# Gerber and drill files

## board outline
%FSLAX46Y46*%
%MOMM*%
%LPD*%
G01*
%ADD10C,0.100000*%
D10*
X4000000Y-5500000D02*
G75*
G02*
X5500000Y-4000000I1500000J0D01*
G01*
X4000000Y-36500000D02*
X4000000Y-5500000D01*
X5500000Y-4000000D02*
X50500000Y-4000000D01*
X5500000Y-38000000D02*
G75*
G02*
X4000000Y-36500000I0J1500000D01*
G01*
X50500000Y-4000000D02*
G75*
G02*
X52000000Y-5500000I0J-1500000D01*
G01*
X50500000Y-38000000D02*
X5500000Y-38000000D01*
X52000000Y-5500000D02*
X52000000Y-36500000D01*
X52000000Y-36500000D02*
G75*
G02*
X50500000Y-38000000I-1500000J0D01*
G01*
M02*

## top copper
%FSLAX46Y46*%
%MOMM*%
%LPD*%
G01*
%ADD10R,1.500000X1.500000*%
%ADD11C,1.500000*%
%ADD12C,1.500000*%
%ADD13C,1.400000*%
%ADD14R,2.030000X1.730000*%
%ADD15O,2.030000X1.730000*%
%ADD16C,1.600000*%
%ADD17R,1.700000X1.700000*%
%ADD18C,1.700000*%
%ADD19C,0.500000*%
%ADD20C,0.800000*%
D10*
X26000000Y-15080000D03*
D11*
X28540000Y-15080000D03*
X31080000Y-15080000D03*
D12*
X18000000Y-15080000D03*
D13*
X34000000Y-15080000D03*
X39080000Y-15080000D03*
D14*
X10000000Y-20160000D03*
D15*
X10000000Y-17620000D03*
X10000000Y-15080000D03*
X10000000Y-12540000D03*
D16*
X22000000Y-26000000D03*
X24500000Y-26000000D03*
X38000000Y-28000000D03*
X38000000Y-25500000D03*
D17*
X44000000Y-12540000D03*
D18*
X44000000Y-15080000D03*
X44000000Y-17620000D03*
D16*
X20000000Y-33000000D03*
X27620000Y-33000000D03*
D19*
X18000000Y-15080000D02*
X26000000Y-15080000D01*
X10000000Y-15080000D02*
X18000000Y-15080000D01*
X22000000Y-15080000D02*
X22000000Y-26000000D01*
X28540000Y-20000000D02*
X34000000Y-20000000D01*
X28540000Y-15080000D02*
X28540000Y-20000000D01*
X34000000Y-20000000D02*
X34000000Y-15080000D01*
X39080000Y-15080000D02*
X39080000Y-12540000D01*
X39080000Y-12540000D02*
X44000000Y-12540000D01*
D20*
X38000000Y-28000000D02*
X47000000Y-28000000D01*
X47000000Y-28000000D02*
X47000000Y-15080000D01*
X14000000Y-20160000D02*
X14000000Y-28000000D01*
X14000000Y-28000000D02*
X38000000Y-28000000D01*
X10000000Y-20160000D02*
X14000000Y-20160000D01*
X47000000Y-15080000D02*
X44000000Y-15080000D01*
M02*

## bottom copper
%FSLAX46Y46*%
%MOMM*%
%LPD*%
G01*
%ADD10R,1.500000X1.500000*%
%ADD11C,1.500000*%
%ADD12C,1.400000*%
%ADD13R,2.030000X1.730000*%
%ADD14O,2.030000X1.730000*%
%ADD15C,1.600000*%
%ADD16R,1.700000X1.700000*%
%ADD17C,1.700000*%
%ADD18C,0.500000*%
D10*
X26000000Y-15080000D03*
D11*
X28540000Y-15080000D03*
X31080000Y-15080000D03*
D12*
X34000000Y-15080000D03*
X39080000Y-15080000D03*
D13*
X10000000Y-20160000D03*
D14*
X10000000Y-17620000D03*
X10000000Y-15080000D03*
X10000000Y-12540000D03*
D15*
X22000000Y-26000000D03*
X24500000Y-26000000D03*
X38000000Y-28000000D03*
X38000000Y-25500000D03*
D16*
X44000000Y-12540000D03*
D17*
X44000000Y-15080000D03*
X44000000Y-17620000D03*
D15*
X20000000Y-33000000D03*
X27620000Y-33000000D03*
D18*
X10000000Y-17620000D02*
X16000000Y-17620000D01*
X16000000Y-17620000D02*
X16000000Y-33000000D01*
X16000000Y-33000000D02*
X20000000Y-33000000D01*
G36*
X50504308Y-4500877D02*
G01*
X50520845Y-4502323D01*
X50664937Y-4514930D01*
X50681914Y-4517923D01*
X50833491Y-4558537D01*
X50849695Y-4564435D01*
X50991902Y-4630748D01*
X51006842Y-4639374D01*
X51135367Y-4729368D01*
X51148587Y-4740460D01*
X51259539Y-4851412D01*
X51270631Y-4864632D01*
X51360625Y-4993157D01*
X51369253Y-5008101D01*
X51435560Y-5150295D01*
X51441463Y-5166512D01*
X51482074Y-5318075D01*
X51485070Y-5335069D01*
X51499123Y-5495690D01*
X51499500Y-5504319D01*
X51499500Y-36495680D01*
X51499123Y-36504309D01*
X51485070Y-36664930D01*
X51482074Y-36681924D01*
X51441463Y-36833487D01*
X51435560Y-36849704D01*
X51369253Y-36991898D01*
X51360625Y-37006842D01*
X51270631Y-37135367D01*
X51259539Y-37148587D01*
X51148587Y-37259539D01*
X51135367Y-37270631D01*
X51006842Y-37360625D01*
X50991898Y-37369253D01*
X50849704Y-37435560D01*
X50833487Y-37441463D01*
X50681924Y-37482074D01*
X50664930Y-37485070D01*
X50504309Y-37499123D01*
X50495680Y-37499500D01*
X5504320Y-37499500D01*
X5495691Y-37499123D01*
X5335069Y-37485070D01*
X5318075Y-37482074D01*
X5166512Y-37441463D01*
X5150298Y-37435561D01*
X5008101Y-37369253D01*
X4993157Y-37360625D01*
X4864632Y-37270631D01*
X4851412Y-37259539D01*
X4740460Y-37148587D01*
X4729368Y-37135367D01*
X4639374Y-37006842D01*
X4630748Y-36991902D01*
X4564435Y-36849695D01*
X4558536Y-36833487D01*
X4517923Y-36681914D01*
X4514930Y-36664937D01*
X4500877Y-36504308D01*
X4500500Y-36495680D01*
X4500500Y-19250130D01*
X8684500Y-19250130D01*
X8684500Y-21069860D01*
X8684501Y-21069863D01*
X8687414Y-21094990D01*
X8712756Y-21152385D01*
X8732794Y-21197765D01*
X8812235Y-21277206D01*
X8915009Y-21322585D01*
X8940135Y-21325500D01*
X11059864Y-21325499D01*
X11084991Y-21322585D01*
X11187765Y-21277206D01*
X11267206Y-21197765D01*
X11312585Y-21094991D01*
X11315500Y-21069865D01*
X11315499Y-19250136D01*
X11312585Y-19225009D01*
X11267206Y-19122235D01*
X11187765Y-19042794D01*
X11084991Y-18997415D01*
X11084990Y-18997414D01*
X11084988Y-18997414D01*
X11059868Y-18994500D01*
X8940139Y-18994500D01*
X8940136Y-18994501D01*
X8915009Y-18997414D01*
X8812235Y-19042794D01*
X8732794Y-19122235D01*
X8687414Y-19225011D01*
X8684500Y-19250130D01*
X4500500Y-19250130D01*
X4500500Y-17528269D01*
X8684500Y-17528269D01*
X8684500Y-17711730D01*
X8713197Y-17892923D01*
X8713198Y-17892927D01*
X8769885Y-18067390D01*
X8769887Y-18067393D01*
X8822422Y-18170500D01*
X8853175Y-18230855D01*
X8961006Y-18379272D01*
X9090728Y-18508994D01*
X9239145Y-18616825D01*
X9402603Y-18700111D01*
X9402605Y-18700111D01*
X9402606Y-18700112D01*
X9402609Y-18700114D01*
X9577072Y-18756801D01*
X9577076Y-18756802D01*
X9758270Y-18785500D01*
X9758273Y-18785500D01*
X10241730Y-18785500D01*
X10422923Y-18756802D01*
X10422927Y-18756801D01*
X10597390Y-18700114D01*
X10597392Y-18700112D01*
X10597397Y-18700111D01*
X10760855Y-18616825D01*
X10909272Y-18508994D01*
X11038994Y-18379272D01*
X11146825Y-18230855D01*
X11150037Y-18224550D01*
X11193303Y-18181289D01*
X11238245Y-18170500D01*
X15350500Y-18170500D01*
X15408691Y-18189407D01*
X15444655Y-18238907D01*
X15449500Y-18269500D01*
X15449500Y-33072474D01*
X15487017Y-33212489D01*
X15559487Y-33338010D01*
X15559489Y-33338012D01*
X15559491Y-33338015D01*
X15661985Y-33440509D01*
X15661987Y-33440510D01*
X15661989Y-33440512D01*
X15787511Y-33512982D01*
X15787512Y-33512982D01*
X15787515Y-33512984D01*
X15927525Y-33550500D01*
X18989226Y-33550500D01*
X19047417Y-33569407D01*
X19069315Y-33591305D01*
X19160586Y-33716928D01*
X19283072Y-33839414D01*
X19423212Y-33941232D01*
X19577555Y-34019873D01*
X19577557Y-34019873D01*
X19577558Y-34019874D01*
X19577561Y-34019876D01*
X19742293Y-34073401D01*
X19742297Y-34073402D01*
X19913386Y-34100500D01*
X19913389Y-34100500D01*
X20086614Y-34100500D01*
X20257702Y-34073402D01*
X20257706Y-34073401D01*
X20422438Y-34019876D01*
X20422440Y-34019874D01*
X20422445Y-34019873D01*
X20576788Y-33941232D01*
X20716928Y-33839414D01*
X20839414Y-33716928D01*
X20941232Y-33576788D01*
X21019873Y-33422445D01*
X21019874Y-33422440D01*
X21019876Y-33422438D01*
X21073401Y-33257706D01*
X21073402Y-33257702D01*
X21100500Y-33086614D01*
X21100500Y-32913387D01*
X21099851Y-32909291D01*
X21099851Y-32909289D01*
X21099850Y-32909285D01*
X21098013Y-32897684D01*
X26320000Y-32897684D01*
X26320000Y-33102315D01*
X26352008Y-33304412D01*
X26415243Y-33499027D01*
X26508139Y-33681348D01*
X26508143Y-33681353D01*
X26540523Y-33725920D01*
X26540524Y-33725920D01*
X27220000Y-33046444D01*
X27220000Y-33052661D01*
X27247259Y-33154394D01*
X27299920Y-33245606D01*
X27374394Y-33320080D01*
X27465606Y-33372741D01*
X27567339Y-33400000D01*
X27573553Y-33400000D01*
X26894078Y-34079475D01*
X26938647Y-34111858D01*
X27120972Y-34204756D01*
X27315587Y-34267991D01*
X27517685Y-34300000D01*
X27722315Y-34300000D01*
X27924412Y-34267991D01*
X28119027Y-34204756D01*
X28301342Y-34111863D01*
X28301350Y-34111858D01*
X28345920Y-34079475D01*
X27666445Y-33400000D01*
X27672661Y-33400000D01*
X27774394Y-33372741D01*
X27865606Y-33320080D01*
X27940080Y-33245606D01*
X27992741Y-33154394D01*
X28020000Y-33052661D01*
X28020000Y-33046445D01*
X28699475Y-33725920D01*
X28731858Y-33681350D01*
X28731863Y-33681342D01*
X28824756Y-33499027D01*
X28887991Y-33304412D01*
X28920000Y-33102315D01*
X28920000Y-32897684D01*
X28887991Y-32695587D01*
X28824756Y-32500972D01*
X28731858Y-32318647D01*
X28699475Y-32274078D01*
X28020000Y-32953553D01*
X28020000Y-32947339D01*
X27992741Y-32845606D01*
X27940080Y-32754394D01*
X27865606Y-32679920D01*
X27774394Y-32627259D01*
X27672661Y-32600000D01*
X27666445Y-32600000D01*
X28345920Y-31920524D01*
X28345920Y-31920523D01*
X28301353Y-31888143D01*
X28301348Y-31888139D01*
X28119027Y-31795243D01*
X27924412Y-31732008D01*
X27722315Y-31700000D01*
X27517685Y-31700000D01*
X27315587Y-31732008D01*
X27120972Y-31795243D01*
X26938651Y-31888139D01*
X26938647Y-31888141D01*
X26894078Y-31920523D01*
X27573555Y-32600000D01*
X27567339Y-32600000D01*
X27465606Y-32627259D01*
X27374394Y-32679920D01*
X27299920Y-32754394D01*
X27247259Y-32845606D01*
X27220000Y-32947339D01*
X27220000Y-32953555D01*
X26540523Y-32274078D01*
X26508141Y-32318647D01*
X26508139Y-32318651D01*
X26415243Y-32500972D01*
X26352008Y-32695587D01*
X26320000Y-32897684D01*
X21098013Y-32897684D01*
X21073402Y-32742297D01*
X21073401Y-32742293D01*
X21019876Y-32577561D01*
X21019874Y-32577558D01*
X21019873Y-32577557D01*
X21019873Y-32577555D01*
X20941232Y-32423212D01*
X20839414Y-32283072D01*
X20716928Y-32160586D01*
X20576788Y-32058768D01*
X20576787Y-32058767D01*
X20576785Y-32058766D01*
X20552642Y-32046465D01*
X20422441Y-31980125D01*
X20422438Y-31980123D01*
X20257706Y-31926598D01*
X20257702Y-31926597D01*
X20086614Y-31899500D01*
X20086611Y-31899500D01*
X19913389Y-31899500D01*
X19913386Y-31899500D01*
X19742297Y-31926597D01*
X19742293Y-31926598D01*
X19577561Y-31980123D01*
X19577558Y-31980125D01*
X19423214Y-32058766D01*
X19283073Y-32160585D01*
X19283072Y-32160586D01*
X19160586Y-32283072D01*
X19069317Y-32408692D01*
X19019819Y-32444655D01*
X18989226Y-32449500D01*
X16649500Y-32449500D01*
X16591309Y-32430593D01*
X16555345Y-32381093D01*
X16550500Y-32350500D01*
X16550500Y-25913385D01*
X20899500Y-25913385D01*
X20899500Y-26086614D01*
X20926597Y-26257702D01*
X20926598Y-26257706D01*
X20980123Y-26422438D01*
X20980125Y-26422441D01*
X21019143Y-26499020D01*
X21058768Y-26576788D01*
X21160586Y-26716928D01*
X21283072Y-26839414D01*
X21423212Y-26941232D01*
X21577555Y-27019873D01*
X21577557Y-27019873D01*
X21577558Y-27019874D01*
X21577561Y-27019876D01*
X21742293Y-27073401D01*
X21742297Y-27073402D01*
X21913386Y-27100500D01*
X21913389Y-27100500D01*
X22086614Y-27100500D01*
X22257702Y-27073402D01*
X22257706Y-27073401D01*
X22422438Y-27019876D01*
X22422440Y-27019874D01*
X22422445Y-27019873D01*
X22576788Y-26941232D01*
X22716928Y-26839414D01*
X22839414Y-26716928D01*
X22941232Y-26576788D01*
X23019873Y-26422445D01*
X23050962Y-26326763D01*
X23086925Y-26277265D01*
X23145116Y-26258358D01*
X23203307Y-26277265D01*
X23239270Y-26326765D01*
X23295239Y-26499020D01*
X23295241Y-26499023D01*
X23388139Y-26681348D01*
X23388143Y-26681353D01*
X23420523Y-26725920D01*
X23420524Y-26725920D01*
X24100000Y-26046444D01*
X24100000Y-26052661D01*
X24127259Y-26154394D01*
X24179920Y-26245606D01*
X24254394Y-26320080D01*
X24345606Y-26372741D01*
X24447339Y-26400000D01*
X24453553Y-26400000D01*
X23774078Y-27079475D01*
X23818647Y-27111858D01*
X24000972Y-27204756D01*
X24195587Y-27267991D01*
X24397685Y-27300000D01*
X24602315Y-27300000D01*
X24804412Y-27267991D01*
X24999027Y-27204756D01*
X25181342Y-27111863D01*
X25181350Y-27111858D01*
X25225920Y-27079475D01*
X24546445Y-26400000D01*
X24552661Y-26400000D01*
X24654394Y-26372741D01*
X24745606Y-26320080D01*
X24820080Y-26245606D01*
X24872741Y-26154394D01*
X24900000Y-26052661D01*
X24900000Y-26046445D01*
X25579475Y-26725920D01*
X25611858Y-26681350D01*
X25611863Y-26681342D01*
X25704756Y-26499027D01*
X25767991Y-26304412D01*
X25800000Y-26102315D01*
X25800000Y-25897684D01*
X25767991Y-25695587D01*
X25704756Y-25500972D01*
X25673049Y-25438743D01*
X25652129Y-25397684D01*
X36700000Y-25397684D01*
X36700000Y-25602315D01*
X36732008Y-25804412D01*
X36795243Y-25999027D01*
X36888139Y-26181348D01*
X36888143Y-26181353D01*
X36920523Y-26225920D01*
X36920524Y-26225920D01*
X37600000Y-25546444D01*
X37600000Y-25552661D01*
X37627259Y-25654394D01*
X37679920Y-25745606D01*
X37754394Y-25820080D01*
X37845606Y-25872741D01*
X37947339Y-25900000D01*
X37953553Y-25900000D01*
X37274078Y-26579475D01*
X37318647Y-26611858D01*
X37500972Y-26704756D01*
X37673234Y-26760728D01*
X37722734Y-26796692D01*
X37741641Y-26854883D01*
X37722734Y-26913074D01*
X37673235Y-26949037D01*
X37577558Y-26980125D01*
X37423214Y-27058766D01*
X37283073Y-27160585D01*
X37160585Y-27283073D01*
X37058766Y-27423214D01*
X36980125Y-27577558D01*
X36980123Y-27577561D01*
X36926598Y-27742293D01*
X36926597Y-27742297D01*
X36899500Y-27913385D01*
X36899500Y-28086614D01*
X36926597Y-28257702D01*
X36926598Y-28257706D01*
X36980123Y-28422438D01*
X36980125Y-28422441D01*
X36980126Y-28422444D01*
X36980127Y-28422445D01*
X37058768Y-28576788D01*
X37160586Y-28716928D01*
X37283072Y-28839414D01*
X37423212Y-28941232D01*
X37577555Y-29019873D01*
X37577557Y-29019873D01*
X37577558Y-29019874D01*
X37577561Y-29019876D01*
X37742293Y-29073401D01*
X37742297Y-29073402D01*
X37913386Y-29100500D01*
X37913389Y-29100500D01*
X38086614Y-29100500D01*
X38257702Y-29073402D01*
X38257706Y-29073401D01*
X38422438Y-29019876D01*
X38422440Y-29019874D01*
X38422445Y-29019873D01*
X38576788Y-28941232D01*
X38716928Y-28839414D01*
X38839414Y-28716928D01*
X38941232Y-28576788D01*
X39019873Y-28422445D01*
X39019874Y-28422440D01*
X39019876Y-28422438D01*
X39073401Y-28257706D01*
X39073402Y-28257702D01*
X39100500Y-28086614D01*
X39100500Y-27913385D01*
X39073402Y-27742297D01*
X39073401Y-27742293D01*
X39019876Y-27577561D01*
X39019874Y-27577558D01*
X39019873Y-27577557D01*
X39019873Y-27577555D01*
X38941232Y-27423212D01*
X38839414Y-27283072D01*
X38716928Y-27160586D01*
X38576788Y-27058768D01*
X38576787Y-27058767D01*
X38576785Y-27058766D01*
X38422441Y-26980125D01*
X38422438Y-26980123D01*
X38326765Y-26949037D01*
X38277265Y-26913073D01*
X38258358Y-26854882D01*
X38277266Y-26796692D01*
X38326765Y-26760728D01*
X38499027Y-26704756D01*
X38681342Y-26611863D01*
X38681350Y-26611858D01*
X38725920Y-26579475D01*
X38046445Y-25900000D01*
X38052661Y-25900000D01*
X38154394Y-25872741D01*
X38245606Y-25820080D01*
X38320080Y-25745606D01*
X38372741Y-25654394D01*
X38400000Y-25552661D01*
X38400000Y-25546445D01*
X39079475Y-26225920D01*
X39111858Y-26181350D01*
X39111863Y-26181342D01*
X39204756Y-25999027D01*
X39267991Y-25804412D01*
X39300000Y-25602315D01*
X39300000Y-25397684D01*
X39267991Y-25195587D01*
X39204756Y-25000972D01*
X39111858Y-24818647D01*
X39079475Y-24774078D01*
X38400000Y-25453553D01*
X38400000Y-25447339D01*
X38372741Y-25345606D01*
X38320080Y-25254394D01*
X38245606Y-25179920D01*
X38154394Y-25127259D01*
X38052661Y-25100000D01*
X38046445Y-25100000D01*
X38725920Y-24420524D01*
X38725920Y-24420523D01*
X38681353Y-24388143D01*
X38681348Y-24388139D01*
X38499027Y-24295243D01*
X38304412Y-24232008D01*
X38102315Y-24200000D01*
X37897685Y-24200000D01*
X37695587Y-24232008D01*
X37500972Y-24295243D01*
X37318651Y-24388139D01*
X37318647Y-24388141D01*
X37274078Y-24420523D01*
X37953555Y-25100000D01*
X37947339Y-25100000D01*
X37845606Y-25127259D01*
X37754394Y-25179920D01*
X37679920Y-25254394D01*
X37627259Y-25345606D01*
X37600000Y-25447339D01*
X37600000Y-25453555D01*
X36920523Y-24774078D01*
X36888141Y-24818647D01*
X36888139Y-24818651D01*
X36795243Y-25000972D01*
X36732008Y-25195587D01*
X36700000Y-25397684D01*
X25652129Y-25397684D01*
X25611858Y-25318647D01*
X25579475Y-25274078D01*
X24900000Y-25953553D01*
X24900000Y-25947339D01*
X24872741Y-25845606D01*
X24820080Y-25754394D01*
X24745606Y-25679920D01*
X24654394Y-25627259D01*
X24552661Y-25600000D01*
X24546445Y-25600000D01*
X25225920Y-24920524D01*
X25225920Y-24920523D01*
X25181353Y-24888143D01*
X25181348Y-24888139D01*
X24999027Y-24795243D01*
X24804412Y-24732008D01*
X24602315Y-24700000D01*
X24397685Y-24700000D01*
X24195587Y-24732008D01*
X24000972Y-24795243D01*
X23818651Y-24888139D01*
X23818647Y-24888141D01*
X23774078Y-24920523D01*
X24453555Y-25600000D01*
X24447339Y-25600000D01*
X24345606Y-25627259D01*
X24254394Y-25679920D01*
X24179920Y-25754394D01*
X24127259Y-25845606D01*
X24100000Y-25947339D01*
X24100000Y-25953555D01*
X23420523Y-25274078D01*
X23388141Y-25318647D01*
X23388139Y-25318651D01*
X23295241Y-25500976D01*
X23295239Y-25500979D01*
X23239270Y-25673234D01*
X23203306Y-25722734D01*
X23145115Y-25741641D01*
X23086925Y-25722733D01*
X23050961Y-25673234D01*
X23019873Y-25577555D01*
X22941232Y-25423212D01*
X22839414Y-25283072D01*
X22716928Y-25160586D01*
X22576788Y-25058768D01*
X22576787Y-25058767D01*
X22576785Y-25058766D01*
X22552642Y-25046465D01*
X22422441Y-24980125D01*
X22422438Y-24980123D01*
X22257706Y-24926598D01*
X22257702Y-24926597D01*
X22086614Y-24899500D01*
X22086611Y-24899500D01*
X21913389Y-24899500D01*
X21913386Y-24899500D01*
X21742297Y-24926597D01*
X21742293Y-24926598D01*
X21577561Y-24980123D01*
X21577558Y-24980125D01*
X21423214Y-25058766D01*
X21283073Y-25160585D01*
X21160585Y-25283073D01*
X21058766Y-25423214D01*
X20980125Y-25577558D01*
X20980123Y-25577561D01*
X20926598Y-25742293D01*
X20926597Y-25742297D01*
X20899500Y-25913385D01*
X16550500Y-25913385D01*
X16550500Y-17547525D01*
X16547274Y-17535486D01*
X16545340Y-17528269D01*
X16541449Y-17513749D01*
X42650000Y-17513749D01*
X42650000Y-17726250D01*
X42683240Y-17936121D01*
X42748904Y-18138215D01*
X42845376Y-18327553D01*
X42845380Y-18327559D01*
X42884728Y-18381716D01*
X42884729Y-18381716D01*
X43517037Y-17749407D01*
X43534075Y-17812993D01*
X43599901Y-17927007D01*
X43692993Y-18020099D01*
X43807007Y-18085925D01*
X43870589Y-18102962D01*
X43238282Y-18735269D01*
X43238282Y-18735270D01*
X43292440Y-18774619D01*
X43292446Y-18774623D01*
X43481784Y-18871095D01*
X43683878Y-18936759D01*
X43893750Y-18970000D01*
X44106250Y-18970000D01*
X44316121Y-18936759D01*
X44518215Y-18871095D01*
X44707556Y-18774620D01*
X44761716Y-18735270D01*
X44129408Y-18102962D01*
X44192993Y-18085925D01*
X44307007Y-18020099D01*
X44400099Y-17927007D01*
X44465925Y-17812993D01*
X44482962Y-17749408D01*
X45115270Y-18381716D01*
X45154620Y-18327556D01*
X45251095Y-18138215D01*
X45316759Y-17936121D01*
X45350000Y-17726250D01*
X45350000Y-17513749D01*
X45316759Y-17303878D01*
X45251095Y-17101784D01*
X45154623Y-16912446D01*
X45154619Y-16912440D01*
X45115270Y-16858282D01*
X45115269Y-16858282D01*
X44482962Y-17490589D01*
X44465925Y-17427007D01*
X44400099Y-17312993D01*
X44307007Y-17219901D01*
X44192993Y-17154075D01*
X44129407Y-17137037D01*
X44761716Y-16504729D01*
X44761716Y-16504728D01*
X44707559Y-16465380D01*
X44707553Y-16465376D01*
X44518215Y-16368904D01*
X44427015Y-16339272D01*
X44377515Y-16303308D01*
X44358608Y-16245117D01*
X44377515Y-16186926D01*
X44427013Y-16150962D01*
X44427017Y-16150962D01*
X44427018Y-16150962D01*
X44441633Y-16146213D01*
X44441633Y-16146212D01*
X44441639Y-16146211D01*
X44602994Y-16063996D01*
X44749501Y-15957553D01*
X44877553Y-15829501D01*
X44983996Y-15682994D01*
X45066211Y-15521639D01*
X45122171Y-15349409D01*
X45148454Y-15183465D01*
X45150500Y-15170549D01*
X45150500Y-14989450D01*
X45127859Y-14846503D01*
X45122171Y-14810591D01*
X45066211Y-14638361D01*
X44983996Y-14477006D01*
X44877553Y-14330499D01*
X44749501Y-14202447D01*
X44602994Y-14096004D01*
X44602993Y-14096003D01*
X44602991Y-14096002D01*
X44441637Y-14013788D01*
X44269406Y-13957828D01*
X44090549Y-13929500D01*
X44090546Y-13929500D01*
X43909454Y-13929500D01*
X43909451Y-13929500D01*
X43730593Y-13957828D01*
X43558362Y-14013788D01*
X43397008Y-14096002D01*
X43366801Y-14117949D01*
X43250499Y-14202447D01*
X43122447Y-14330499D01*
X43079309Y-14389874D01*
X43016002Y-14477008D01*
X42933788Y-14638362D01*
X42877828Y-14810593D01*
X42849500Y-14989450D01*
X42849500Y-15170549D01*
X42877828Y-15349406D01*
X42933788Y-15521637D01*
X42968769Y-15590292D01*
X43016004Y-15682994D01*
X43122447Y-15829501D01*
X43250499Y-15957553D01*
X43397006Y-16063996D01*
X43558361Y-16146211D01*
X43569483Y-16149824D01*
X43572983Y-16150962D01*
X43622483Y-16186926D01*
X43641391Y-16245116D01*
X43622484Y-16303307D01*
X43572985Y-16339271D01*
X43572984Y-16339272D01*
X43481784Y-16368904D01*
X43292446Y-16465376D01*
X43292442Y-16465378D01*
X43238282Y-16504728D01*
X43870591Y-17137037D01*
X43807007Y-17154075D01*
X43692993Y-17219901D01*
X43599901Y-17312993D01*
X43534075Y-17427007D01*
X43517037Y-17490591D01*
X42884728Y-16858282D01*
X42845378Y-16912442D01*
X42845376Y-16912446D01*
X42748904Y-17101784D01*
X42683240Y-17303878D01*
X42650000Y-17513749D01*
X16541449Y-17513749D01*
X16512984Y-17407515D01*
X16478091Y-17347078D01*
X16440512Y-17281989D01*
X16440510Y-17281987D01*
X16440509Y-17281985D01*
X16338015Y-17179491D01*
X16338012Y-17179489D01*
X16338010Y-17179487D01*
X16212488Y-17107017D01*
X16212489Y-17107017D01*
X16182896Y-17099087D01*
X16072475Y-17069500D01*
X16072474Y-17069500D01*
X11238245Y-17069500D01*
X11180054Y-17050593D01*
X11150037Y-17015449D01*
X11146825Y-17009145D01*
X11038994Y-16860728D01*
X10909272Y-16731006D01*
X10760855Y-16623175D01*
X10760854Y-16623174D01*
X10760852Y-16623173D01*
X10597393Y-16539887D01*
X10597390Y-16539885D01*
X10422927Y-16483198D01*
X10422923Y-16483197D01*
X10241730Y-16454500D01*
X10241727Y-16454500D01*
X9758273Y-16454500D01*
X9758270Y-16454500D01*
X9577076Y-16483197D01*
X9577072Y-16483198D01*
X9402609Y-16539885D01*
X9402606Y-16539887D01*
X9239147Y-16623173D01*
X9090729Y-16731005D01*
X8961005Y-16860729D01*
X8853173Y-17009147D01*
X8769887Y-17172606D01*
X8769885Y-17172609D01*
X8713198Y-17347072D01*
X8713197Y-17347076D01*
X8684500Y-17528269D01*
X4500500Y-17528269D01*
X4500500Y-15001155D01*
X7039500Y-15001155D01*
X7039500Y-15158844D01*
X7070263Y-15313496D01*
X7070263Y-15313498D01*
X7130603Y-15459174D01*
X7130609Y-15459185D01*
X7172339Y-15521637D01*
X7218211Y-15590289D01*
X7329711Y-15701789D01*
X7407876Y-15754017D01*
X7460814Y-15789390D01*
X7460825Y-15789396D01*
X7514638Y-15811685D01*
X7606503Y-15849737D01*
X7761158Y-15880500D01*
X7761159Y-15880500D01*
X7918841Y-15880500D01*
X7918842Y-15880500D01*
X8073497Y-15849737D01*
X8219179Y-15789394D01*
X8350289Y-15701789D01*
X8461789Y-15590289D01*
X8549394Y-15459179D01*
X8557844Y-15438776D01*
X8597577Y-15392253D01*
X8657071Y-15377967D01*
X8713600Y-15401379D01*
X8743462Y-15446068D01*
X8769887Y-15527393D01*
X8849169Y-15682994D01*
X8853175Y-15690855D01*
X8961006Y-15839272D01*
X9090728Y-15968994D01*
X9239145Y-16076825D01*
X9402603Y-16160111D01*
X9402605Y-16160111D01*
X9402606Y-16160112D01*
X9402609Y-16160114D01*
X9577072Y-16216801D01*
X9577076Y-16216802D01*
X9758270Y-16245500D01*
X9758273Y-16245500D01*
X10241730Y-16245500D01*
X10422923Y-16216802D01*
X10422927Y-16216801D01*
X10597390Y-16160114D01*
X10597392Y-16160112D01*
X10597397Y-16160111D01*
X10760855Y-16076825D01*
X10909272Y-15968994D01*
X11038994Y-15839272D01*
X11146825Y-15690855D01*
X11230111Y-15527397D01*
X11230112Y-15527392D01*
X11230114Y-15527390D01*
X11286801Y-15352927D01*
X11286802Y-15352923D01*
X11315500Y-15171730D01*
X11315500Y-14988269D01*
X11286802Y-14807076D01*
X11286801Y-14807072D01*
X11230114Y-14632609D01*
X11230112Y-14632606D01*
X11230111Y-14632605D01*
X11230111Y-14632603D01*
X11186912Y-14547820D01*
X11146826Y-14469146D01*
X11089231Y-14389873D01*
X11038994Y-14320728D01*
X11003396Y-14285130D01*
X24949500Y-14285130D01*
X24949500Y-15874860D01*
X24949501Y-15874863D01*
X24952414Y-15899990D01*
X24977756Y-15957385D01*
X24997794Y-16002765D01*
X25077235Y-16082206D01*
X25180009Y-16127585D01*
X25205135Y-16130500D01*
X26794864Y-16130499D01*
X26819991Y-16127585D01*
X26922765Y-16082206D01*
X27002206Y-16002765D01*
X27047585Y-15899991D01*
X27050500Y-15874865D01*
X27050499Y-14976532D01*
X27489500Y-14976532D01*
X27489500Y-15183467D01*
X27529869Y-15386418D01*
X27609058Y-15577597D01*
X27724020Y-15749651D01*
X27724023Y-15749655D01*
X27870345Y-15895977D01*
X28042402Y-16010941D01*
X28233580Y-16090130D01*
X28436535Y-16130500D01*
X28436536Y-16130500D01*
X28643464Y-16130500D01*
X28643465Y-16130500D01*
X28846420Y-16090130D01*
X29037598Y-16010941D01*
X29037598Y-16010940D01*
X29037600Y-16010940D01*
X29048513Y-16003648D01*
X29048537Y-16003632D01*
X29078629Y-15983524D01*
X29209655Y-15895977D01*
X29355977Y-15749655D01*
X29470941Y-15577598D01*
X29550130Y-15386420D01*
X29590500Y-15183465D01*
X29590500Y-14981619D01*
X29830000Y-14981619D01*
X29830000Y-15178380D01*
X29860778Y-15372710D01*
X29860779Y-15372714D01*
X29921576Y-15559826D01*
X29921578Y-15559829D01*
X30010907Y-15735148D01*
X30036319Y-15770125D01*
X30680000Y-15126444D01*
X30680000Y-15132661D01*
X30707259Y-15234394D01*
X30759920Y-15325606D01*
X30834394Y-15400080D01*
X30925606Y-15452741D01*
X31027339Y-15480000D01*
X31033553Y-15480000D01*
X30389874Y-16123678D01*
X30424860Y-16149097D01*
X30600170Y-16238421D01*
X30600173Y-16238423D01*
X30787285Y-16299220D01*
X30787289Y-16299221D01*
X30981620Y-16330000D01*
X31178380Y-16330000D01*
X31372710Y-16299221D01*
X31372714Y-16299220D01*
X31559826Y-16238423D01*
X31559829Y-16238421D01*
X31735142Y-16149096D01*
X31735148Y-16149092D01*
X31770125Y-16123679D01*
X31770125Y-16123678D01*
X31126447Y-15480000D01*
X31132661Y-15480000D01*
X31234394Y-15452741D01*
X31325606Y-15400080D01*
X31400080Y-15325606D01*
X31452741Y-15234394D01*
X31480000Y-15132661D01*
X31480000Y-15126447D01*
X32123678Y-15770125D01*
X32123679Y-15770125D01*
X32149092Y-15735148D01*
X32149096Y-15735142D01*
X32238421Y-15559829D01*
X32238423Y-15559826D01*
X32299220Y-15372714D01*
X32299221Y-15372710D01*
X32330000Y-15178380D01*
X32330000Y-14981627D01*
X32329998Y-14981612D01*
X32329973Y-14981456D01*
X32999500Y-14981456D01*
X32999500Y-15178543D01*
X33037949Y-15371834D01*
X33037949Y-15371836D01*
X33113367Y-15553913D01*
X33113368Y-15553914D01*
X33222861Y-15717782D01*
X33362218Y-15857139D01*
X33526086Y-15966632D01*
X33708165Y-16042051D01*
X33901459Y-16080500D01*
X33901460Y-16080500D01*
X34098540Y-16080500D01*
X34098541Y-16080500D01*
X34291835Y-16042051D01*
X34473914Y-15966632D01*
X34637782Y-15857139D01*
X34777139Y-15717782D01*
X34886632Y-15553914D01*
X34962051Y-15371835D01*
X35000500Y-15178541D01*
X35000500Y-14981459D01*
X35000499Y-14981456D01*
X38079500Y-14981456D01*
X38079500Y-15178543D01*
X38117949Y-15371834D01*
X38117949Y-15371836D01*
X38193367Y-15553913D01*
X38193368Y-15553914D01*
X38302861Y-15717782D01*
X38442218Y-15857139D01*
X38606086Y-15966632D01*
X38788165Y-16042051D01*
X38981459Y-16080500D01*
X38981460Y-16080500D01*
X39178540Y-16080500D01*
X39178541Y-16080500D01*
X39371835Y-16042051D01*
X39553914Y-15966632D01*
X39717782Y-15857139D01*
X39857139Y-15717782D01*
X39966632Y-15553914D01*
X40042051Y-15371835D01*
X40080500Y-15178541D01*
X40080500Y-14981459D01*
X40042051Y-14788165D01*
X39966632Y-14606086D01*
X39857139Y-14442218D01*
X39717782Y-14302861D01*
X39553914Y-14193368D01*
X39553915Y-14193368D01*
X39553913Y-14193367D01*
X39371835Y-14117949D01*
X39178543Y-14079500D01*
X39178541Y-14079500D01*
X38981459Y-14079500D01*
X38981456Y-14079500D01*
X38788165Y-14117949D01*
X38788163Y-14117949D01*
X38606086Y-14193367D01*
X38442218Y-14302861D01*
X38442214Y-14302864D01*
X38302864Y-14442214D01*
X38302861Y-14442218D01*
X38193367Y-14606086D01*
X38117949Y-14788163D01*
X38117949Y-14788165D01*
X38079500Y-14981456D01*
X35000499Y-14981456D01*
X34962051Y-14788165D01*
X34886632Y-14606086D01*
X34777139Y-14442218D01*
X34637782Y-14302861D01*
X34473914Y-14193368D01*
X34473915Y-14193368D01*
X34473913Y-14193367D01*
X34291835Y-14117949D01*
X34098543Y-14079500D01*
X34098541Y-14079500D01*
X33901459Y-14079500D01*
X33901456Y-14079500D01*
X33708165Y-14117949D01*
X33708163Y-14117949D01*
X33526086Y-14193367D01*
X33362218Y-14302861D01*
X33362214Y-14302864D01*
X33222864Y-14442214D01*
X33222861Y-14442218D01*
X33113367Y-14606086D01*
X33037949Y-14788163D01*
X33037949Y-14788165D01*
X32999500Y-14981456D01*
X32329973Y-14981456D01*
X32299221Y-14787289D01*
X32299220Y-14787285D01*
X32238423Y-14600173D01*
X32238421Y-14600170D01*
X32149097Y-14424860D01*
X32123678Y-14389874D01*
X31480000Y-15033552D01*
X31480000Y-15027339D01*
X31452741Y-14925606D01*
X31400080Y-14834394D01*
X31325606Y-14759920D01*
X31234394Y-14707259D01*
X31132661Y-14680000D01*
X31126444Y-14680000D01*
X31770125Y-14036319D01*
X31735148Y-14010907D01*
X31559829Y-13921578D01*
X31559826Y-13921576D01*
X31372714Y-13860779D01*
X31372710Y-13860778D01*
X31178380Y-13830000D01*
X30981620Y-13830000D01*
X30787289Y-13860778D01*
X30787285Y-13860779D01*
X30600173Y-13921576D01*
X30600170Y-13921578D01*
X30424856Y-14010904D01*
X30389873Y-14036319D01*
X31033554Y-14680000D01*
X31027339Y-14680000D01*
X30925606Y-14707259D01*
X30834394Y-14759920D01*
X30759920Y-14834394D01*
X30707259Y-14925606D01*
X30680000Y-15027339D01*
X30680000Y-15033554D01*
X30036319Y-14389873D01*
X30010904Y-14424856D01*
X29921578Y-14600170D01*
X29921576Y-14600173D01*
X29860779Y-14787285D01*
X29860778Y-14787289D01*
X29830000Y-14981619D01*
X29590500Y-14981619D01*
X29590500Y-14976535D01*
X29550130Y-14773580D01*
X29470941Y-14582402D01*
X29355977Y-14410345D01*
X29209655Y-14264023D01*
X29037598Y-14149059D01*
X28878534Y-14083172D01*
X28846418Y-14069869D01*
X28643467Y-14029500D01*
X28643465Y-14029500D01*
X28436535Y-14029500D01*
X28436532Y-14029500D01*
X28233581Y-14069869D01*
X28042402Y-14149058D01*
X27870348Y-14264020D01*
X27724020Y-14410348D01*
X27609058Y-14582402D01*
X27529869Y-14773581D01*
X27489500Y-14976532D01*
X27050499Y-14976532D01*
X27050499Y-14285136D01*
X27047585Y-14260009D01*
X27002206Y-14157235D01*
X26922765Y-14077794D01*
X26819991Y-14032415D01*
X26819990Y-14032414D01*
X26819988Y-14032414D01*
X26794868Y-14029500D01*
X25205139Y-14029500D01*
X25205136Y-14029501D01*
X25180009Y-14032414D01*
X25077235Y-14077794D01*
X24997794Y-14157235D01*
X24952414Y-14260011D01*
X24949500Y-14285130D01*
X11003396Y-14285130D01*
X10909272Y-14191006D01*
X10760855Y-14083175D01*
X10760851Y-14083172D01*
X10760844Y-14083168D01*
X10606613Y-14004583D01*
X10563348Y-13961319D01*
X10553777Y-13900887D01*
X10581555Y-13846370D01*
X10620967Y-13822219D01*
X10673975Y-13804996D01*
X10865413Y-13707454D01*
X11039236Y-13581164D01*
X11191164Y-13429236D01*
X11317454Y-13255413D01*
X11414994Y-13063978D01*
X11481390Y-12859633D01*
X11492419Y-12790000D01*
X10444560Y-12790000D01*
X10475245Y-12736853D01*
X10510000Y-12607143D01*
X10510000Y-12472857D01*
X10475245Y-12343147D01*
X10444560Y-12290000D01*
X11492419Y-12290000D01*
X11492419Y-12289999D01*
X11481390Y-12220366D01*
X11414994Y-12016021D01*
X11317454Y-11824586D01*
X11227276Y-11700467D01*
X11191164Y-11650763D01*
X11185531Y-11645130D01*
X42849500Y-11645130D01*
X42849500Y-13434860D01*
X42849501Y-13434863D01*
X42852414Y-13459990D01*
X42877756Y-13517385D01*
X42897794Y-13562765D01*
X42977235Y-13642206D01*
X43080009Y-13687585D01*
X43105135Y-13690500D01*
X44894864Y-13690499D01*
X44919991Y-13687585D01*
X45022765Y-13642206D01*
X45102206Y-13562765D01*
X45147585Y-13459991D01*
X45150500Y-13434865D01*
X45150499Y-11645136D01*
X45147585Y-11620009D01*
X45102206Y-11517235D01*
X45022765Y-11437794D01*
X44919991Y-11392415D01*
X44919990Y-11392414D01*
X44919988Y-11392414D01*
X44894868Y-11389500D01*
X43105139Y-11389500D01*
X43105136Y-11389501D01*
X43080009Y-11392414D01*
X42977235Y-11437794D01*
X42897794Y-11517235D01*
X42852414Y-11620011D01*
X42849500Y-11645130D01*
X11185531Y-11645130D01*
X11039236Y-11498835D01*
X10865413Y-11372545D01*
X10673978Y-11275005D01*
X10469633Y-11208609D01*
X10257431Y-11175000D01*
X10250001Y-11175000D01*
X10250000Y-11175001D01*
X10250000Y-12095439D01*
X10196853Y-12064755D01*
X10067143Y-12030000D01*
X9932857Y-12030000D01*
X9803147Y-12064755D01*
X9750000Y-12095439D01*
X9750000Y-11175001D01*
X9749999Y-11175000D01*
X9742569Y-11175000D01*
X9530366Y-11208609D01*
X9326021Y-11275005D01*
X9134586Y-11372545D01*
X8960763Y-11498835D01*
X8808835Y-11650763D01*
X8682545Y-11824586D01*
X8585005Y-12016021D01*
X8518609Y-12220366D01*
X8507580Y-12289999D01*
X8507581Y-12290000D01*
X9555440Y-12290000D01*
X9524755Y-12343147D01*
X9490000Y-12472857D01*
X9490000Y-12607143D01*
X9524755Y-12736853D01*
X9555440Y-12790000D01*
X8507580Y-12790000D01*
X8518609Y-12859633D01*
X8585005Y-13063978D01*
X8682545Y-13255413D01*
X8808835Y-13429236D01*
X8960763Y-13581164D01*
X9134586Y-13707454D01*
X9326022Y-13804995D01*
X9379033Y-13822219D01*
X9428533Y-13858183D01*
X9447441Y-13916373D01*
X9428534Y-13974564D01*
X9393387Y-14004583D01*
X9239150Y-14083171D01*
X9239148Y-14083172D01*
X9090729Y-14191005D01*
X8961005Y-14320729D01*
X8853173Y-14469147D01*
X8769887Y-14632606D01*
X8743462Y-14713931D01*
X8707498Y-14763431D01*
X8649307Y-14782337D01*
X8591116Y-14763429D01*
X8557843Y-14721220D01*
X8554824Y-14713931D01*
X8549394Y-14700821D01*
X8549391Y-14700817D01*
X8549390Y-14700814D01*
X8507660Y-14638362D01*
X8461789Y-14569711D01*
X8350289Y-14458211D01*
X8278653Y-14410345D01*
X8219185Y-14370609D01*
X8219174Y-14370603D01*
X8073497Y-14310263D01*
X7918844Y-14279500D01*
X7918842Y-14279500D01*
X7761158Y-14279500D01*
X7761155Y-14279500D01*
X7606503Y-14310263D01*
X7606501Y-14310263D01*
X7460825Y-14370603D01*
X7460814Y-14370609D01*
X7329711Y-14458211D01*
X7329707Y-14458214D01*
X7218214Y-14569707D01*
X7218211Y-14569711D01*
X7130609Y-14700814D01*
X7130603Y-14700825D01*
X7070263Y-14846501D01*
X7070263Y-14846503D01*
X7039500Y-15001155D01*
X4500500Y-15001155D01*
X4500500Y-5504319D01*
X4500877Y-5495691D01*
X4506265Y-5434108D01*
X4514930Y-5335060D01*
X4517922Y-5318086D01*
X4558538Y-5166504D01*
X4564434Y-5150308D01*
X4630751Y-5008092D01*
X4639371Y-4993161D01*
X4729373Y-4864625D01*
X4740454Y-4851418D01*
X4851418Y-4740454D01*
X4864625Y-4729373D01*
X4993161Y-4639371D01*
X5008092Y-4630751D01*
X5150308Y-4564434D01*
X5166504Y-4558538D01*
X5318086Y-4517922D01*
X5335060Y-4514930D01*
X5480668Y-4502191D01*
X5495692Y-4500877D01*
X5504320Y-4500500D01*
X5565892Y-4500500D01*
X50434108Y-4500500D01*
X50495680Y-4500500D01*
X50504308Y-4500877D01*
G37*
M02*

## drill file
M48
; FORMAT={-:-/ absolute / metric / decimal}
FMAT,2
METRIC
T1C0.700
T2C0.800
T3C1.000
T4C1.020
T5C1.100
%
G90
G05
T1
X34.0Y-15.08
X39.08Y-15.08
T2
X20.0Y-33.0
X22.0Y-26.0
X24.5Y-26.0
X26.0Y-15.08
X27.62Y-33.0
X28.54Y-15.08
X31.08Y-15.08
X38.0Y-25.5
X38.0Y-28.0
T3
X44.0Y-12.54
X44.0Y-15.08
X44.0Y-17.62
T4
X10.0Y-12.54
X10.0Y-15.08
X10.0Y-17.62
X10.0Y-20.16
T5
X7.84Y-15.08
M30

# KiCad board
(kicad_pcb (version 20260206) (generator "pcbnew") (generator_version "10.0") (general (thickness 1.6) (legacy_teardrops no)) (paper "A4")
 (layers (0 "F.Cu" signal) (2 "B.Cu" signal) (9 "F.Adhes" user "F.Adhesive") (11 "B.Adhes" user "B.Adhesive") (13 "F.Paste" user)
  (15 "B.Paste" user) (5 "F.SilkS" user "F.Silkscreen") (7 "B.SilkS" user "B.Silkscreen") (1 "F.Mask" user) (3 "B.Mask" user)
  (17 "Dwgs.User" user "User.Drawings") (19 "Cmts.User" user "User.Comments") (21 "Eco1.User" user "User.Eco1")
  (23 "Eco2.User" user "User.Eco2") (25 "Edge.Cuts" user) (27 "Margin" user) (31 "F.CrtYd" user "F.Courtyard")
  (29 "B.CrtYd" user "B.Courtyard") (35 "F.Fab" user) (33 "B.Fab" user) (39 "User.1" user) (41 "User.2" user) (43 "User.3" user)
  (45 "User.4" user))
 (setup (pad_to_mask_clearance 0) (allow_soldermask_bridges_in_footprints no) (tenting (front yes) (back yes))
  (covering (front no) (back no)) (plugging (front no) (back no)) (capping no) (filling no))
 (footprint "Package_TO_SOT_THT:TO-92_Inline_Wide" (layer "F.Cu") (at 26 15.08)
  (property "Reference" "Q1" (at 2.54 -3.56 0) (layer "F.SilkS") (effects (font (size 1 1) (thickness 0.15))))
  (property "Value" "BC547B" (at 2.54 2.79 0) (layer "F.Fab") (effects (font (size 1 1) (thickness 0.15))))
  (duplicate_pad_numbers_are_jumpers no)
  (pad "1" thru_hole rect (at 0 0) (size 1.5 1.5) (drill 0.8) (layers "*.Cu" "*.Mask") (remove_unused_layers no) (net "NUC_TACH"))
  (pad "2" thru_hole circle (at 2.54 0) (size 1.5 1.5) (drill 0.8) (layers "*.Cu" "*.Mask") (remove_unused_layers no) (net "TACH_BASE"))
  (pad "3" thru_hole circle (at 5.08 0) (size 1.5 1.5) (drill 0.8) (layers "*.Cu" "*.Mask") (remove_unused_layers no) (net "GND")))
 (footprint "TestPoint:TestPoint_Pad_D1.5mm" (layer "F.Cu") (at 18 15.08)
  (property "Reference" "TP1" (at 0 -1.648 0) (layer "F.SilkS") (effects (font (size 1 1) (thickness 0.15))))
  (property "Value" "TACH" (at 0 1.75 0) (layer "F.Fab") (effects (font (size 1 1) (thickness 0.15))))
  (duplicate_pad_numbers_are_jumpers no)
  (pad "1" smd circle (at 0 0) (size 1.5 1.5) (layers "F.Cu" "F.Mask") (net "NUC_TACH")))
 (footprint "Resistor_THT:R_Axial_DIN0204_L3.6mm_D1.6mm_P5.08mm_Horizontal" (layer "F.Cu") (at 34 15.08)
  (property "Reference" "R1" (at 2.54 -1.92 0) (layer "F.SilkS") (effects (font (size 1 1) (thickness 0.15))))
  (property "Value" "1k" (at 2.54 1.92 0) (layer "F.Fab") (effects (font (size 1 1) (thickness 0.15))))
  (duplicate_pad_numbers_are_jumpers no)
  (pad "1" thru_hole circle (at 0 0) (size 1.4 1.4) (drill 0.7) (layers "*.Cu" "*.Mask") (remove_unused_layers no) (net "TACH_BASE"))
  (pad "2" thru_hole circle (at 5.08 0) (size 1.4 1.4) (drill 0.7) (layers "*.Cu" "*.Mask") (remove_unused_layers no) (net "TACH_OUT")))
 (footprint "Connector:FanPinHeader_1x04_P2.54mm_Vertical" (layer "F.Cu") (at 10 20.16 90)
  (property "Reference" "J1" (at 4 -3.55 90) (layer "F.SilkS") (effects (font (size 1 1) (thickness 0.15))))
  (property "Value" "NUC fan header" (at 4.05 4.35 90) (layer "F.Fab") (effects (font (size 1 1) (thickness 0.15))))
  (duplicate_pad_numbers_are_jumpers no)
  (pad "" np_thru_hole circle (at 5.08 -2.16 180) (size 1.1 1.1) (drill 1.1) (layers "*.Cu" "*.Mask"))
  (pad "1" thru_hole rect (at 0 0 180) (size 2.03 1.73) (drill 1.02) (layers "*.Cu" "*.Mask") (remove_unused_layers no) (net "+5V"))
  (pad "2" thru_hole oval (at 2.54 0 180) (size 2.03 1.73) (drill 1.02) (layers "*.Cu" "*.Mask") (remove_unused_layers no) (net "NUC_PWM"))
  (pad "3" thru_hole oval (at 5.08 0 180) (size 2.03 1.73) (drill 1.02) (layers "*.Cu" "*.Mask") (remove_unused_layers no) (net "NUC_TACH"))
  (pad "4" thru_hole oval (at 7.62 0 180) (size 2.03 1.73) (drill 1.02) (layers "*.Cu" "*.Mask") (remove_unused_layers no) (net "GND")))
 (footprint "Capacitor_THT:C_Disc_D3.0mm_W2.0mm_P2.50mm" (layer "F.Cu") (at 22 26)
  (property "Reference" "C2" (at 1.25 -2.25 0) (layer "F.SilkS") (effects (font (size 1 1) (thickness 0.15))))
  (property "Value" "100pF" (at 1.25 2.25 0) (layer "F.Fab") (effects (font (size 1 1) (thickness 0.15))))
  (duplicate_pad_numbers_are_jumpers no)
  (pad "1" thru_hole circle (at 0 0) (size 1.6 1.6) (drill 0.8) (layers "*.Cu" "*.Mask") (remove_unused_layers no) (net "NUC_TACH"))
  (pad "2" thru_hole circle (at 2.5 0) (size 1.6 1.6) (drill 0.8) (layers "*.Cu" "*.Mask") (remove_unused_layers no) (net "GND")))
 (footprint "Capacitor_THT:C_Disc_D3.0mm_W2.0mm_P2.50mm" (layer "F.Cu") (at 38 28 90)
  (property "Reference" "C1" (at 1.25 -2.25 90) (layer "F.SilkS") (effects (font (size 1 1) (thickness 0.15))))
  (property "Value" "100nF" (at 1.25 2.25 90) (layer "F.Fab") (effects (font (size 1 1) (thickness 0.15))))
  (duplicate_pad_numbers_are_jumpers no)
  (pad "1" thru_hole circle (at 0 0 90) (size 1.6 1.6) (drill 0.8) (layers "*.Cu" "*.Mask") (remove_unused_layers no) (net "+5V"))
  (pad "2" thru_hole circle (at 2.5 0 90) (size 1.6 1.6) (drill 0.8) (layers "*.Cu" "*.Mask") (remove_unused_layers no) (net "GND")))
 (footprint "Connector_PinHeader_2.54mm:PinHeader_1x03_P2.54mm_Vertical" (layer "F.Cu") (at 44 12.54)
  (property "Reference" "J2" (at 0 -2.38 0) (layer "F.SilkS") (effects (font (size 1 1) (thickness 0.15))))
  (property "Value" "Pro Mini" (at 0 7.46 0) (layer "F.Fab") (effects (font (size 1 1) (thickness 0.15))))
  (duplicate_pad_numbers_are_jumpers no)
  (pad "1" thru_hole rect (at 0 0) (size 1.7 1.7) (drill 1) (layers "*.Cu" "*.Mask") (remove_unused_layers no) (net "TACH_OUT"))
  (pad "2" thru_hole circle (at 0 2.54) (size 1.7 1.7) (drill 1) (layers "*.Cu" "*.Mask") (remove_unused_layers no) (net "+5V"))
  (pad "3" thru_hole circle (at 0 5.08) (size 1.7 1.7) (drill 1) (layers "*.Cu" "*.Mask") (remove_unused_layers no) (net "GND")))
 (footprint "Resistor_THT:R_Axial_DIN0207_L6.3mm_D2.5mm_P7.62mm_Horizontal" (layer "F.Cu") (at 20 33)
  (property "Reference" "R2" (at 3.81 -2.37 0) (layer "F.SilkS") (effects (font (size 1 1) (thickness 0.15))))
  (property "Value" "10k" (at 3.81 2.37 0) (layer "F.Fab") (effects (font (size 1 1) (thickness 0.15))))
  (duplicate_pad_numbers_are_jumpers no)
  (pad "1" thru_hole circle (at 0 0) (size 1.6 1.6) (drill 0.8) (layers "*.Cu" "*.Mask") (remove_unused_layers no) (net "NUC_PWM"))
  (pad "2" thru_hole circle (at 7.62 0) (size 1.6 1.6) (drill 0.8) (layers "*.Cu" "*.Mask") (remove_unused_layers no) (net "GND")))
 (gr_arc (start 4 5.5) (mid 4.43934 4.43934) (end 5.5 4) (stroke (width 0.1) (type default)) (layer "Edge.Cuts"))
 (gr_line (start 4 36.5) (end 4 5.5) (stroke (width 0.1) (type default)) (layer "Edge.Cuts"))
 (gr_line (start 5.5 4) (end 50.5 4) (stroke (width 0.1) (type default)) (layer "Edge.Cuts"))
 (gr_arc (start 5.5 38) (mid 4.43934 37.56066) (end 4 36.5) (stroke (width 0.1) (type default)) (layer "Edge.Cuts"))
 (gr_arc (start 50.5 4) (mid 51.56066 4.43934) (end 52 5.5) (stroke (width 0.1) (type default)) (layer "Edge.Cuts"))
 (gr_line (start 50.5 38) (end 5.5 38) (stroke (width 0.1) (type default)) (layer "Edge.Cuts"))
 (gr_line (start 52 5.5) (end 52 36.5) (stroke (width 0.1) (type default)) (layer "Edge.Cuts"))
 (gr_arc (start 52 36.5) (mid 51.56066 37.56066) (end 50.5 38) (stroke (width 0.1) (type default)) (layer "Edge.Cuts"))
 (segment (start 18 15.08) (end 26 15.08) (width 0.5) (layer "F.Cu") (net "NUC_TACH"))
 (segment (start 10 15.08) (end 18 15.08) (width 0.5) (layer "F.Cu") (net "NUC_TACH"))
 (segment (start 22 15.08) (end 22 26) (width 0.5) (layer "F.Cu") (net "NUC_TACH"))
 (segment (start 28.54 20) (end 34 20) (width 0.5) (layer "F.Cu") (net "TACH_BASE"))
 (segment (start 28.54 15.08) (end 28.54 20) (width 0.5) (layer "F.Cu") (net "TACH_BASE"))
 (segment (start 34 20) (end 34 15.08) (width 0.5) (layer "F.Cu") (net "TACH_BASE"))
 (segment (start 39.08 15.08) (end 39.08 12.54) (width 0.5) (layer "F.Cu") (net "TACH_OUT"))
 (segment (start 39.08 12.54) (end 44 12.54) (width 0.5) (layer "F.Cu") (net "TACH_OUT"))
 (segment (start 38 28) (end 47 28) (width 0.8) (layer "F.Cu") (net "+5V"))
 (segment (start 47 28) (end 47 15.08) (width 0.8) (layer "F.Cu") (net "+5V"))
 (segment (start 14 20.16) (end 14 28) (width 0.8) (layer "F.Cu") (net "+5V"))
 (segment (start 14 28) (end 38 28) (width 0.8) (layer "F.Cu") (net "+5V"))
 (segment (start 10 20.16) (end 14 20.16) (width 0.8) (layer "F.Cu") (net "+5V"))
 (segment (start 47 15.08) (end 44 15.08) (width 0.8) (layer "F.Cu") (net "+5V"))
 (segment (start 10 17.62) (end 16 17.62) (width 0.5) (layer "B.Cu") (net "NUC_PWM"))
 (segment (start 16 17.62) (end 16 33) (width 0.5) (layer "B.Cu") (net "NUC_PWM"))
 (segment (start 16 33) (end 20 33) (width 0.5) (layer "B.Cu") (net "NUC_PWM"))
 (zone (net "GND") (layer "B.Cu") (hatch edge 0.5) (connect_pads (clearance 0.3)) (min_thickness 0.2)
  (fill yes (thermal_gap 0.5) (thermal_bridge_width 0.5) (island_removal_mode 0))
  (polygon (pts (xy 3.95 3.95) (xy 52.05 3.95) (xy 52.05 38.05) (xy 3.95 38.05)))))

